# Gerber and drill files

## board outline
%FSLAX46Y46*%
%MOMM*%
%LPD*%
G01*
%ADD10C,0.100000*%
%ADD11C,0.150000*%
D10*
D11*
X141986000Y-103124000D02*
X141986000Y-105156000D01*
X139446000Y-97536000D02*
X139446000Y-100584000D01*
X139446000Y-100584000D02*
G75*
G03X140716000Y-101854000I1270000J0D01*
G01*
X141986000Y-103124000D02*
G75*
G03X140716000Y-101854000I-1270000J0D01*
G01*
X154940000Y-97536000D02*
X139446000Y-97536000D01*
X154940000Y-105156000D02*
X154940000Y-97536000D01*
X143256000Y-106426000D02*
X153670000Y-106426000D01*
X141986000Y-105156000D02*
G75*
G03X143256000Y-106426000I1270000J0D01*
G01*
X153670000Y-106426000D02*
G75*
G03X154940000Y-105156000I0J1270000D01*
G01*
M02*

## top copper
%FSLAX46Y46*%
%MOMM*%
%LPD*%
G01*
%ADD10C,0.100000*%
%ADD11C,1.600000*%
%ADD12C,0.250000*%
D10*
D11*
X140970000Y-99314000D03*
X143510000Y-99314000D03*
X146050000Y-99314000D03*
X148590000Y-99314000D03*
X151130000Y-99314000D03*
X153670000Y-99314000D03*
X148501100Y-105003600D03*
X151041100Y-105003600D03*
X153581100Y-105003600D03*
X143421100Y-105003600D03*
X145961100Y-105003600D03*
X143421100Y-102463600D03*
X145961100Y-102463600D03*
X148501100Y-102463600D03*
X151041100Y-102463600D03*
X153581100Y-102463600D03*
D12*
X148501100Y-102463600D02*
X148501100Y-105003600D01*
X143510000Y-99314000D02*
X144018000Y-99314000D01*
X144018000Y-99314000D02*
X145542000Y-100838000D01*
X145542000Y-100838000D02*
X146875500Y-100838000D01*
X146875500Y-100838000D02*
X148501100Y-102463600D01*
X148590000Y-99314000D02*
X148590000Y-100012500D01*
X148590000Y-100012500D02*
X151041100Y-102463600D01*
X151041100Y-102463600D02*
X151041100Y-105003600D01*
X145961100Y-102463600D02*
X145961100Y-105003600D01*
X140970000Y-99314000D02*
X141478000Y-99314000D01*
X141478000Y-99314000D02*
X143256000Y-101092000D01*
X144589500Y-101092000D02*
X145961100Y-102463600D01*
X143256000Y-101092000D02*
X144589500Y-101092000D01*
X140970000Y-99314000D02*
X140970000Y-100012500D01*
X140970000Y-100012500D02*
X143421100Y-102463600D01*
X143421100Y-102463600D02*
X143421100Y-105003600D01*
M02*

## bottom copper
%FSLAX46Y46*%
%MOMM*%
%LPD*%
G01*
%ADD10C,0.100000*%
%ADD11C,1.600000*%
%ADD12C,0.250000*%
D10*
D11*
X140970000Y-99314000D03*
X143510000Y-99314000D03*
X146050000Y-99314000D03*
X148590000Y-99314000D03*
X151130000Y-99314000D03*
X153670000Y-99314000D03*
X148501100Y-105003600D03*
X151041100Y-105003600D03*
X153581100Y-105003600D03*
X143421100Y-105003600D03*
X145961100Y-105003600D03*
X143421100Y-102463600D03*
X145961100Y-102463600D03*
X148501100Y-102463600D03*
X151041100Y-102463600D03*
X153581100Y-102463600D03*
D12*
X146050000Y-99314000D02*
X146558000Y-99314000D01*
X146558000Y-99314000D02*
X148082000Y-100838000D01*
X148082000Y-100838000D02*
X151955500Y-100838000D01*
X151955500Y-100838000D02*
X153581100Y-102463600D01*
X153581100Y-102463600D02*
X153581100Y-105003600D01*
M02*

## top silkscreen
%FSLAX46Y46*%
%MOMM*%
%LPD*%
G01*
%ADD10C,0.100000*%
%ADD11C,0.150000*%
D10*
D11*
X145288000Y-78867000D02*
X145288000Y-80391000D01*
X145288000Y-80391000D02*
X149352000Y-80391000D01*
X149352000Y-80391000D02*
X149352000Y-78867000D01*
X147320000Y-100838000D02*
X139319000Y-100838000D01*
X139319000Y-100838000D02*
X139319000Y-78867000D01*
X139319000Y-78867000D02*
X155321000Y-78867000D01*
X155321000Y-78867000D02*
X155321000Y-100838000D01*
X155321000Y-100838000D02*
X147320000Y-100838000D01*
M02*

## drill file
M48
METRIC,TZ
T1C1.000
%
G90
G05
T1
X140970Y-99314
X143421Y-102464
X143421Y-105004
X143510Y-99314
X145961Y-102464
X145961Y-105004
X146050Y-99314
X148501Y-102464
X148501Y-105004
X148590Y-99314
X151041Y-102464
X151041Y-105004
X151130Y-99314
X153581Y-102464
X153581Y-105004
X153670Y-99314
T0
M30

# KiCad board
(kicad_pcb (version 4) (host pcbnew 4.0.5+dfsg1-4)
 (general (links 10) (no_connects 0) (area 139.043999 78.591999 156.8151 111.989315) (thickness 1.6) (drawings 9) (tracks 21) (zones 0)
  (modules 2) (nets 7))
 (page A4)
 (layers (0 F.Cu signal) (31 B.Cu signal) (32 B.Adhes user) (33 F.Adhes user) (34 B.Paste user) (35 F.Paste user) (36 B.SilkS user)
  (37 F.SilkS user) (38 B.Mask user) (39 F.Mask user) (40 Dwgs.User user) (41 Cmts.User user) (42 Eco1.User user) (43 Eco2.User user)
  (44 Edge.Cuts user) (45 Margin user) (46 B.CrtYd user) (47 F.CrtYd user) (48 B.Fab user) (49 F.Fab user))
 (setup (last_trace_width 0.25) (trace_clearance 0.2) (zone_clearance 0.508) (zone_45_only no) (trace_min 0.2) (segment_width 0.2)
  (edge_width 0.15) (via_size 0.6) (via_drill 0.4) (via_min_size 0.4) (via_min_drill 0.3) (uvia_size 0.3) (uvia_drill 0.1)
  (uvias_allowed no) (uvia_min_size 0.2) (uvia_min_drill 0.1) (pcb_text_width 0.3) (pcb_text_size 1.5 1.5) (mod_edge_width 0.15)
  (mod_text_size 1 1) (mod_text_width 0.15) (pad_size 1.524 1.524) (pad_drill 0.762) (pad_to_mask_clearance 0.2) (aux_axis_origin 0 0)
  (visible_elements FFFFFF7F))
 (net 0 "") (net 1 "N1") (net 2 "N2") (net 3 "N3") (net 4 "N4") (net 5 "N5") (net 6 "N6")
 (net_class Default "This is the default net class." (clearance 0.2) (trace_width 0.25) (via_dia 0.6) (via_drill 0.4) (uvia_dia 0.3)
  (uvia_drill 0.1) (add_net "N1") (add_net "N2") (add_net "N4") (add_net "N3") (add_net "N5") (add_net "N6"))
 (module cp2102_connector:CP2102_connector (layer F.Cu) (at 147.32 99.314)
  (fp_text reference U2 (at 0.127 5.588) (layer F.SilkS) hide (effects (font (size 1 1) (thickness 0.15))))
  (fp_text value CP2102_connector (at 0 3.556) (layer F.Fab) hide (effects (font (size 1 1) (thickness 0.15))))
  (fp_line (start -2.032 -20.447) (end -2.032 -18.923) (layer F.SilkS) (width 0.15))
  (fp_line (start -2.032 -18.923) (end 2.032 -18.923) (layer F.SilkS) (width 0.15))
  (fp_line (start 2.032 -18.923) (end 2.032 -20.447) (layer F.SilkS) (width 0.15))
  (fp_line (start 0 1.524) (end -8.001 1.524) (layer F.SilkS) (width 0.15))
  (fp_line (start -8.001 1.524) (end -8.001 -20.447) (layer F.SilkS) (width 0.15))
  (fp_line (start -8.001 -20.447) (end 8.001 -20.447) (layer F.SilkS) (width 0.15))
  (fp_line (start 8.001 -20.447) (end 8.001 1.524) (layer F.SilkS) (width 0.15))
  (fp_line (start 8.001 1.524) (end 0 1.524) (layer F.SilkS) (width 0.15))
  (pad 1 thru_hole circle (at -6.35 0) (size 1.6 1.6) (drill 1) (layers *.Cu *.Mask) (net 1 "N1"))
  (pad 2 thru_hole circle (at -3.81 0) (size 1.6 1.6) (drill 1) (layers *.Cu *.Mask) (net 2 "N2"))
  (pad 3 thru_hole circle (at -1.27 0) (size 1.6 1.6) (drill 1) (layers *.Cu *.Mask) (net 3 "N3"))
  (pad 4 thru_hole circle (at 1.27 0) (size 1.6 1.6) (drill 1) (layers *.Cu *.Mask) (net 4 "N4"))
  (pad 5 thru_hole circle (at 3.81 0) (size 1.6 1.6) (drill 1) (layers *.Cu *.Mask) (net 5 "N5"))
  (pad 6 thru_hole circle (at 6.35 0) (size 1.6 1.6) (drill 1) (layers *.Cu *.Mask) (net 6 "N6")))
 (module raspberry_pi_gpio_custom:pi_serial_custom (layer F.Cu) (at 148.5011 105.0036)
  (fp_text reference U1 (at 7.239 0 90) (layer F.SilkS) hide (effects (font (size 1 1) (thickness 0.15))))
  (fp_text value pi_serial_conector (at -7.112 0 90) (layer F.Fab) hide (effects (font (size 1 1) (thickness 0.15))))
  (pad 3 thru_hole circle (at 0 0) (size 1.6 1.6) (drill 1) (layers *.Cu *.Mask) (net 2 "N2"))
  (pad 4 thru_hole circle (at 2.54 0) (size 1.6 1.6) (drill 1) (layers *.Cu *.Mask) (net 4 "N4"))
  (pad 5 thru_hole circle (at 5.08 0) (size 1.6 1.6) (drill 1) (layers *.Cu *.Mask) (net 3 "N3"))
  (pad 1 thru_hole circle (at -5.08 0) (size 1.6 1.6) (drill 1) (layers *.Cu *.Mask) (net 1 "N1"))
  (pad 2 thru_hole circle (at -2.54 0) (size 1.6 1.6) (drill 1) (layers *.Cu *.Mask) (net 1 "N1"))
  (pad 1 thru_hole circle (at -5.08 -2.54) (size 1.6 1.6) (drill 1) (layers *.Cu *.Mask) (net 1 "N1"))
  (pad 2 thru_hole circle (at -2.54 -2.54) (size 1.6 1.6) (drill 1) (layers *.Cu *.Mask) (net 1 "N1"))
  (pad 3 thru_hole circle (at 0 -2.54) (size 1.6 1.6) (drill 1) (layers *.Cu *.Mask) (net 2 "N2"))
  (pad 4 thru_hole circle (at 2.54 -2.54) (size 1.6 1.6) (drill 1) (layers *.Cu *.Mask) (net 4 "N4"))
  (pad 5 thru_hole circle (at 5.08 -2.54) (size 1.6 1.6) (drill 1) (layers *.Cu *.Mask) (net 3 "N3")))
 (gr_line (start 141.986 103.124) (end 141.986 105.156) (angle 90) (layer Edge.Cuts) (width 0.15))
 (gr_line (start 139.446 97.536) (end 139.446 100.584) (angle 90) (layer Edge.Cuts) (width 0.15))
 (gr_arc (start 140.716 100.584) (end 140.716 101.854) (angle 90) (layer Edge.Cuts) (width 0.15))
 (gr_arc (start 140.716 103.124) (end 140.716 101.854) (angle 90) (layer Edge.Cuts) (width 0.15))
 (gr_line (start 154.94 97.536) (end 139.446 97.536) (angle 90) (layer Edge.Cuts) (width 0.15))
 (gr_line (start 154.94 105.156) (end 154.94 97.536) (angle 90) (layer Edge.Cuts) (width 0.15))
 (gr_line (start 143.256 106.426) (end 153.67 106.426) (angle 90) (layer Edge.Cuts) (width 0.15))
 (gr_arc (start 143.256 105.156) (end 143.256 106.426) (angle 90) (layer Edge.Cuts) (width 0.15))
 (gr_arc (start 153.67 105.156) (end 154.94 105.156) (angle 90) (layer Edge.Cuts) (width 0.15))
 (segment (start 148.5011 102.4636) (end 148.5011 105.0036) (width 0.25) (layer F.Cu) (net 2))
 (segment (start 143.51 99.314) (end 144.018 99.314) (width 0.25) (layer F.Cu) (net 2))
 (segment (start 144.018 99.314) (end 145.542 100.838) (width 0.25) (layer F.Cu) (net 2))
 (segment (start 145.542 100.838) (end 146.8755 100.838) (width 0.25) (layer F.Cu) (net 2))
 (segment (start 146.8755 100.838) (end 148.5011 102.4636) (width 0.25) (layer F.Cu) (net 2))
 (segment (start 148.59 99.314) (end 148.59 100.0125) (width 0.25) (layer F.Cu) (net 4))
 (segment (start 148.59 100.0125) (end 151.0411 102.4636) (width 0.25) (layer F.Cu) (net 4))
 (segment (start 151.0411 102.4636) (end 151.0411 105.0036) (width 0.25) (layer F.Cu) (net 4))
 (segment (start 146.05 99.314) (end 146.558 99.314) (width 0.25) (layer B.Cu) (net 3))
 (segment (start 146.558 99.314) (end 148.082 100.838) (width 0.25) (layer B.Cu) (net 3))
 (segment (start 148.082 100.838) (end 151.9555 100.838) (width 0.25) (layer B.Cu) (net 3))
 (segment (start 151.9555 100.838) (end 153.5811 102.4636) (width 0.25) (layer B.Cu) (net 3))
 (segment (start 153.5811 102.4636) (end 153.5811 105.0036) (width 0.25) (layer B.Cu) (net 3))
 (segment (start 145.9611 102.4636) (end 145.9611 105.0036) (width 0.25) (layer F.Cu) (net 1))
 (segment (start 140.97 99.314) (end 141.478 99.314) (width 0.25) (layer F.Cu) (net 1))
 (segment (start 141.478 99.314) (end 143.256 101.092) (width 0.25) (layer F.Cu) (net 1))
 (segment (start 144.5895 101.092) (end 145.9611 102.4636) (width 0.25) (layer F.Cu) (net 1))
 (segment (start 143.256 101.092) (end 144.5895 101.092) (width 0.25) (layer F.Cu) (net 1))
 (segment (start 140.97 99.314) (end 140.97 100.0125) (width 0.25) (layer F.Cu) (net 1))
 (segment (start 140.97 100.0125) (end 143.4211 102.4636) (width 0.25) (layer F.Cu) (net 1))
 (segment (start 143.4211 102.4636) (end 143.4211 105.0036) (width 0.25) (layer F.Cu) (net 1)))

